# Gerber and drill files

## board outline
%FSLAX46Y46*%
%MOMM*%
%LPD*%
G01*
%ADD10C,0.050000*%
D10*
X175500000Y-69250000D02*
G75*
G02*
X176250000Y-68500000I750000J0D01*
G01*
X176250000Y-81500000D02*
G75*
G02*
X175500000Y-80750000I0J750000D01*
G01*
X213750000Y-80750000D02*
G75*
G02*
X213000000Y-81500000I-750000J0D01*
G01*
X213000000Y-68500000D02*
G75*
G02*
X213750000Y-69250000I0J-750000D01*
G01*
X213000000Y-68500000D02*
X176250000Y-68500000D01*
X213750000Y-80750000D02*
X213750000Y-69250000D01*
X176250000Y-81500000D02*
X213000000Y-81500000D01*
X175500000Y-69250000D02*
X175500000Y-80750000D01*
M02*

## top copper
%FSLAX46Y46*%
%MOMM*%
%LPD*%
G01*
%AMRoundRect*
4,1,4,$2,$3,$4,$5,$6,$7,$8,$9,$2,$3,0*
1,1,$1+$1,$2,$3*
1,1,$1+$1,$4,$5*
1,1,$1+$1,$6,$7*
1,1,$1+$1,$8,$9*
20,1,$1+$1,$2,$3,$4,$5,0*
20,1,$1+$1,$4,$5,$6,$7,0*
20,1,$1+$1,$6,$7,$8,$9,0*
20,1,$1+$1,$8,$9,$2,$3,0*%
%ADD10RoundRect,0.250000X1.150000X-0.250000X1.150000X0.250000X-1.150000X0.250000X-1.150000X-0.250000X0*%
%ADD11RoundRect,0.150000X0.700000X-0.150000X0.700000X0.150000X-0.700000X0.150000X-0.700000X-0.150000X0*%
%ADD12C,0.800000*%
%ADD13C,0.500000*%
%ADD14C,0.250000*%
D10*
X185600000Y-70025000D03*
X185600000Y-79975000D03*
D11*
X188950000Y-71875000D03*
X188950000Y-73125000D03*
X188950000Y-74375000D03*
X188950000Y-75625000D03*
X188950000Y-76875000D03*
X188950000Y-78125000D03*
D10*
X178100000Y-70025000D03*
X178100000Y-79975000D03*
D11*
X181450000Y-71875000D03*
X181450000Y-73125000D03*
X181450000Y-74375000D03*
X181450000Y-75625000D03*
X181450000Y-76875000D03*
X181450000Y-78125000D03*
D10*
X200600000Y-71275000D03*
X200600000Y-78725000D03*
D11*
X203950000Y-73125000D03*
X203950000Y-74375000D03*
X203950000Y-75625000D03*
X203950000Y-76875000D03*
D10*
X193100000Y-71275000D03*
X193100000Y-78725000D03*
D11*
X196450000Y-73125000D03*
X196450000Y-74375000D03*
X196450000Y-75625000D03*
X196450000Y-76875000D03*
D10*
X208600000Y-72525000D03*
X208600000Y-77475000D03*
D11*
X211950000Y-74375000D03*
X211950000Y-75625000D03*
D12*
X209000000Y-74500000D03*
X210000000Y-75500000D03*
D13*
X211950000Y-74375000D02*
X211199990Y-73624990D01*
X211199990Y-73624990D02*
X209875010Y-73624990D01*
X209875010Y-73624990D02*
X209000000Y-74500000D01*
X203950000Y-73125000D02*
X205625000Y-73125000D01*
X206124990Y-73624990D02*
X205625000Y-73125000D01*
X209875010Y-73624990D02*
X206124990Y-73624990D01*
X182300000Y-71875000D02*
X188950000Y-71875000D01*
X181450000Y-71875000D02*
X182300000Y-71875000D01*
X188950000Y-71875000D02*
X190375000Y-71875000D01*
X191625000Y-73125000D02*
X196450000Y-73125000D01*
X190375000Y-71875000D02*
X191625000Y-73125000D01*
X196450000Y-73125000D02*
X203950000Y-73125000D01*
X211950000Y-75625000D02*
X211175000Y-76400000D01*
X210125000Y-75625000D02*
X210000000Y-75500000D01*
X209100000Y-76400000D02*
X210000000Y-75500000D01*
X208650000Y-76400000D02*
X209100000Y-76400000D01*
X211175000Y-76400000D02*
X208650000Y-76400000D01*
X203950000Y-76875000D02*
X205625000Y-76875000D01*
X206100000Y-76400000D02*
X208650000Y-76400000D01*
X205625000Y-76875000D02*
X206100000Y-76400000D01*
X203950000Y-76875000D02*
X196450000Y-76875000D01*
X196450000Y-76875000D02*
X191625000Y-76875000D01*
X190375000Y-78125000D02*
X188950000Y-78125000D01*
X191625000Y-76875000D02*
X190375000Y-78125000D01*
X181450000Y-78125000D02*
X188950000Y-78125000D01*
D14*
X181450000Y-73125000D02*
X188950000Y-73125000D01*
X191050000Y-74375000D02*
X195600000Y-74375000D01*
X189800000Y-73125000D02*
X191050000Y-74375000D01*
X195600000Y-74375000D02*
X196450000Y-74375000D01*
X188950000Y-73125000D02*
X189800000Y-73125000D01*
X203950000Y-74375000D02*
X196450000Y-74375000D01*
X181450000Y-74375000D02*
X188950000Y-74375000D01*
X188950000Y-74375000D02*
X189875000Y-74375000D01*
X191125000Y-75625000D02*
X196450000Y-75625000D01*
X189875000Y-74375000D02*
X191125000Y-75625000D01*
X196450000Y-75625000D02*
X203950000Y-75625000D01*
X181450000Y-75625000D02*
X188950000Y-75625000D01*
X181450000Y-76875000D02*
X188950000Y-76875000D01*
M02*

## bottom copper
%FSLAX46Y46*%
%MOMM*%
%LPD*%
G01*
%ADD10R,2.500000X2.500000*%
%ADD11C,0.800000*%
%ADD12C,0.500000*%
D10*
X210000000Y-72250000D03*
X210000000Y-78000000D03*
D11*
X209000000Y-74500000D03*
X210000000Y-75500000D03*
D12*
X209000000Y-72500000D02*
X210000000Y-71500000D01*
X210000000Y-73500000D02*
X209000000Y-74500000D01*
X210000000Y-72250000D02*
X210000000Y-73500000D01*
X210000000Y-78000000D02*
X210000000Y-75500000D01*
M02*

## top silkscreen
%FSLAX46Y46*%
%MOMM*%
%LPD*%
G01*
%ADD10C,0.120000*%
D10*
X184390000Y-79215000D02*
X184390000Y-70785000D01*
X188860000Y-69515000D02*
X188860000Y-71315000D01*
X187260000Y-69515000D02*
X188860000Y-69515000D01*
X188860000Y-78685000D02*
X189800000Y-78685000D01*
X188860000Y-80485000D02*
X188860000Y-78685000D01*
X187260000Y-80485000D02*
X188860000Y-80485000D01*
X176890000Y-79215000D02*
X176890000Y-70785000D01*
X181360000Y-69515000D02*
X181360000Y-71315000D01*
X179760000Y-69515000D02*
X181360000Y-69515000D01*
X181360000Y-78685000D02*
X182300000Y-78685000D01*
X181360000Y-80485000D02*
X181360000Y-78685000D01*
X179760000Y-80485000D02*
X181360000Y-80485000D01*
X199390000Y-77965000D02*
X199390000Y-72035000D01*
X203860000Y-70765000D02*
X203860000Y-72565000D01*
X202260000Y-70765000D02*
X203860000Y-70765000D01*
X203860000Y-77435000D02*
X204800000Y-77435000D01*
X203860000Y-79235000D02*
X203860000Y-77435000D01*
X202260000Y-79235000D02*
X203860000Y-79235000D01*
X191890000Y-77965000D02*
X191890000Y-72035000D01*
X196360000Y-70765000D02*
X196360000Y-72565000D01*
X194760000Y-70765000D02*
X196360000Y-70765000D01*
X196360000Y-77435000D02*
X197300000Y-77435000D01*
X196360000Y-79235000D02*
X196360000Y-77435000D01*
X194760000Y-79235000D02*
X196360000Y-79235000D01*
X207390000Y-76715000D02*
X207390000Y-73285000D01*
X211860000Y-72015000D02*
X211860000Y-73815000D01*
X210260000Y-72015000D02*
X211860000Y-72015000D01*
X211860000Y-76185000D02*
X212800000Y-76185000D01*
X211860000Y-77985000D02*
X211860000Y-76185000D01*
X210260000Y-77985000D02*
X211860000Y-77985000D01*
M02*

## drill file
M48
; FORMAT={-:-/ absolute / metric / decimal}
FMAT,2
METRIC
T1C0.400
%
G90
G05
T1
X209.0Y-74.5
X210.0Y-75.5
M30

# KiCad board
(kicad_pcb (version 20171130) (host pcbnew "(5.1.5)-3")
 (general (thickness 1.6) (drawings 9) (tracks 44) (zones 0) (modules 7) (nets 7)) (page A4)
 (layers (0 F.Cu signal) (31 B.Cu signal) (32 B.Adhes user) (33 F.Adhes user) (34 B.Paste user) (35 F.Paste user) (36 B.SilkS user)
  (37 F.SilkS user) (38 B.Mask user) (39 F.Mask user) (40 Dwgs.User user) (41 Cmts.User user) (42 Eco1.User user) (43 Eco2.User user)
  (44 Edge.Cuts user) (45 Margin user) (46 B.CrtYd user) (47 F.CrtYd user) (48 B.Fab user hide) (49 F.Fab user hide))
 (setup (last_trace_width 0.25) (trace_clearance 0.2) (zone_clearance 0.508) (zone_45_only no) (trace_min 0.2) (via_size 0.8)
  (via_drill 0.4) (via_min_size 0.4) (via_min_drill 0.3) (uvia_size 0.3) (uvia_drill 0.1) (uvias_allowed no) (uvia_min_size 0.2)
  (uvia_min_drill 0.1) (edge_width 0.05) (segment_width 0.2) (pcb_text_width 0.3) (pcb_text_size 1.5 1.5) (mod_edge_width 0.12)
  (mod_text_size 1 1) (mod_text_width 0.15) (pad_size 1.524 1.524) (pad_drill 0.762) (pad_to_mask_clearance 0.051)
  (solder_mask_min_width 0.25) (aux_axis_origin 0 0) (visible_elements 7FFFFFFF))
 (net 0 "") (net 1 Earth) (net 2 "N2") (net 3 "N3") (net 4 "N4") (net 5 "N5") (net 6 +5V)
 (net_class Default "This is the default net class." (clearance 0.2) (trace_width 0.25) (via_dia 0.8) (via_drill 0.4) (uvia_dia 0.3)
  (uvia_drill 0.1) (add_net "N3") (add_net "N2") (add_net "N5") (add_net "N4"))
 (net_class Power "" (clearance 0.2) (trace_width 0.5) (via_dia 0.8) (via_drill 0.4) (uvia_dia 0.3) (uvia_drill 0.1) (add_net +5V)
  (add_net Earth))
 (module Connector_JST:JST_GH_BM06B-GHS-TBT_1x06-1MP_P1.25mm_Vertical (layer F.Cu) (at 187 75 90)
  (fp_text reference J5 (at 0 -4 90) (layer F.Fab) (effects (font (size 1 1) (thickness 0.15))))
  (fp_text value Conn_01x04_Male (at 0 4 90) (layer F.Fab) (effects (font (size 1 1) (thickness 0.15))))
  (fp_line (start -4.215 -2.61) (end 4.215 -2.61) (layer F.SilkS) (width 0.12))
  (fp_line (start 5.485 1.86) (end 3.685 1.86) (layer F.SilkS) (width 0.12))
  (fp_line (start 5.485 0.26) (end 5.485 1.86) (layer F.SilkS) (width 0.12))
  (fp_line (start -3.685 1.86) (end -3.685 2.8) (layer F.SilkS) (width 0.12))
  (fp_line (start -5.485 1.86) (end -3.685 1.86) (layer F.SilkS) (width 0.12))
  (fp_line (start -5.485 0.26) (end -5.485 1.86) (layer F.SilkS) (width 0.12))
  (pad MP smd roundrect (at 4.975 -1.4 90) (size 1 2.8) (layers F.Cu F.Paste F.Mask) (roundrect_rratio 0.25))
  (pad MP smd roundrect (at -4.975 -1.4 90) (size 1 2.8) (layers F.Cu F.Paste F.Mask) (roundrect_rratio 0.25))
  (pad 6 smd roundrect (at 3.125 1.95 90) (size 0.6 1.7) (layers F.Cu F.Paste F.Mask) (roundrect_rratio 0.25) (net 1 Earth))
  (pad 5 smd roundrect (at 1.875 1.95 90) (size 0.6 1.7) (layers F.Cu F.Paste F.Mask) (roundrect_rratio 0.25) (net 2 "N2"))
  (pad 4 smd roundrect (at 0.625 1.95 90) (size 0.6 1.7) (layers F.Cu F.Paste F.Mask) (roundrect_rratio 0.25) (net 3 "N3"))
  (pad 3 smd roundrect (at -0.625 1.95 90) (size 0.6 1.7) (layers F.Cu F.Paste F.Mask) (roundrect_rratio 0.25) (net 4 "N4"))
  (pad 2 smd roundrect (at -1.875 1.95 90) (size 0.6 1.7) (layers F.Cu F.Paste F.Mask) (roundrect_rratio 0.25) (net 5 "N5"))
  (pad 1 smd roundrect (at -3.125 1.95 90) (size 0.6 1.7) (layers F.Cu F.Paste F.Mask) (roundrect_rratio 0.25) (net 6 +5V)))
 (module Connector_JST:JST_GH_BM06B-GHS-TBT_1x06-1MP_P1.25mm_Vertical (layer F.Cu) (at 179.5 75 90)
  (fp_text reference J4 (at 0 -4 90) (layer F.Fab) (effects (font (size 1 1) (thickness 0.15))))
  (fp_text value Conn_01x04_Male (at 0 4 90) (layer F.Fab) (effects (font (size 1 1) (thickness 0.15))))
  (fp_line (start -4.215 -2.61) (end 4.215 -2.61) (layer F.SilkS) (width 0.12))
  (fp_line (start 5.485 1.86) (end 3.685 1.86) (layer F.SilkS) (width 0.12))
  (fp_line (start 5.485 0.26) (end 5.485 1.86) (layer F.SilkS) (width 0.12))
  (fp_line (start -3.685 1.86) (end -3.685 2.8) (layer F.SilkS) (width 0.12))
  (fp_line (start -5.485 1.86) (end -3.685 1.86) (layer F.SilkS) (width 0.12))
  (fp_line (start -5.485 0.26) (end -5.485 1.86) (layer F.SilkS) (width 0.12))
  (pad MP smd roundrect (at 4.975 -1.4 90) (size 1 2.8) (layers F.Cu F.Paste F.Mask) (roundrect_rratio 0.25))
  (pad MP smd roundrect (at -4.975 -1.4 90) (size 1 2.8) (layers F.Cu F.Paste F.Mask) (roundrect_rratio 0.25))
  (pad 6 smd roundrect (at 3.125 1.95 90) (size 0.6 1.7) (layers F.Cu F.Paste F.Mask) (roundrect_rratio 0.25) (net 1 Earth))
  (pad 5 smd roundrect (at 1.875 1.95 90) (size 0.6 1.7) (layers F.Cu F.Paste F.Mask) (roundrect_rratio 0.25) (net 2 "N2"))
  (pad 4 smd roundrect (at 0.625 1.95 90) (size 0.6 1.7) (layers F.Cu F.Paste F.Mask) (roundrect_rratio 0.25) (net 3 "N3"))
  (pad 3 smd roundrect (at -0.625 1.95 90) (size 0.6 1.7) (layers F.Cu F.Paste F.Mask) (roundrect_rratio 0.25) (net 4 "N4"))
  (pad 2 smd roundrect (at -1.875 1.95 90) (size 0.6 1.7) (layers F.Cu F.Paste F.Mask) (roundrect_rratio 0.25) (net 5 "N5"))
  (pad 1 smd roundrect (at -3.125 1.95 90) (size 0.6 1.7) (layers F.Cu F.Paste F.Mask) (roundrect_rratio 0.25) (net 6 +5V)))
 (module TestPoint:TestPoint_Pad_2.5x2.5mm (layer B.Cu) (at 210 72.25)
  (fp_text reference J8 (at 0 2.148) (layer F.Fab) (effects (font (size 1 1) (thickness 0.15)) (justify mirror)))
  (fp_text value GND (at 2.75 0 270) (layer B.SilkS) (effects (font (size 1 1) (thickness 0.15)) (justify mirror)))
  (pad 1 smd rect (at 0 0) (size 2.5 2.5) (layers B.Cu B.Mask) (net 1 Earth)))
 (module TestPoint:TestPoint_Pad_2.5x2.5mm (layer B.Cu) (at 210 78)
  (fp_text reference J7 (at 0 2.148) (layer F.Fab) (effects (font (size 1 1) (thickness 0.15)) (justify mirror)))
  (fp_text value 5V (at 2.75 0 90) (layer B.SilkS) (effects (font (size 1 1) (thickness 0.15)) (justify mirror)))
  (pad 1 smd rect (at 0 0) (size 2.5 2.5) (layers B.Cu B.Mask) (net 6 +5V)))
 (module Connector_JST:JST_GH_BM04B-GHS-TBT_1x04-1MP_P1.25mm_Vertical (layer F.Cu) (at 202 75 90)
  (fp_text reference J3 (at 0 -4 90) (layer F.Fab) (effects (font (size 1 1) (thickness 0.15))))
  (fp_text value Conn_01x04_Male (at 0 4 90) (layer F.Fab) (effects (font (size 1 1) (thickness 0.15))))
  (fp_line (start -2.965 -2.61) (end 2.965 -2.61) (layer F.SilkS) (width 0.12))
  (fp_line (start 4.235 1.86) (end 2.435 1.86) (layer F.SilkS) (width 0.12))
  (fp_line (start 4.235 0.26) (end 4.235 1.86) (layer F.SilkS) (width 0.12))
  (fp_line (start -2.435 1.86) (end -2.435 2.8) (layer F.SilkS) (width 0.12))
  (fp_line (start -4.235 1.86) (end -2.435 1.86) (layer F.SilkS) (width 0.12))
  (fp_line (start -4.235 0.26) (end -4.235 1.86) (layer F.SilkS) (width 0.12))
  (pad MP smd roundrect (at 3.725 -1.4 90) (size 1 2.8) (layers F.Cu F.Paste F.Mask) (roundrect_rratio 0.25))
  (pad MP smd roundrect (at -3.725 -1.4 90) (size 1 2.8) (layers F.Cu F.Paste F.Mask) (roundrect_rratio 0.25))
  (pad 4 smd roundrect (at 1.875 1.95 90) (size 0.6 1.7) (layers F.Cu F.Paste F.Mask) (roundrect_rratio 0.25) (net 1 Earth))
  (pad 3 smd roundrect (at 0.625 1.95 90) (size 0.6 1.7) (layers F.Cu F.Paste F.Mask) (roundrect_rratio 0.25) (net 2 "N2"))
  (pad 2 smd roundrect (at -0.625 1.95 90) (size 0.6 1.7) (layers F.Cu F.Paste F.Mask) (roundrect_rratio 0.25) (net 3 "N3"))
  (pad 1 smd roundrect (at -1.875 1.95 90) (size 0.6 1.7) (layers F.Cu F.Paste F.Mask) (roundrect_rratio 0.25) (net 6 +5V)))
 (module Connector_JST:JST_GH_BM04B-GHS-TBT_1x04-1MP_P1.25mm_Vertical (layer F.Cu) (at 194.5 75 90)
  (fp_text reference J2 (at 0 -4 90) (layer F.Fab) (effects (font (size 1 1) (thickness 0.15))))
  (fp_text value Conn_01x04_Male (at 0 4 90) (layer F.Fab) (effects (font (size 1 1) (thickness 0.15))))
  (fp_line (start -2.965 -2.61) (end 2.965 -2.61) (layer F.SilkS) (width 0.12))
  (fp_line (start 4.235 1.86) (end 2.435 1.86) (layer F.SilkS) (width 0.12))
  (fp_line (start 4.235 0.26) (end 4.235 1.86) (layer F.SilkS) (width 0.12))
  (fp_line (start -2.435 1.86) (end -2.435 2.8) (layer F.SilkS) (width 0.12))
  (fp_line (start -4.235 1.86) (end -2.435 1.86) (layer F.SilkS) (width 0.12))
  (fp_line (start -4.235 0.26) (end -4.235 1.86) (layer F.SilkS) (width 0.12))
  (pad MP smd roundrect (at 3.725 -1.4 90) (size 1 2.8) (layers F.Cu F.Paste F.Mask) (roundrect_rratio 0.25))
  (pad MP smd roundrect (at -3.725 -1.4 90) (size 1 2.8) (layers F.Cu F.Paste F.Mask) (roundrect_rratio 0.25))
  (pad 4 smd roundrect (at 1.875 1.95 90) (size 0.6 1.7) (layers F.Cu F.Paste F.Mask) (roundrect_rratio 0.25) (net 1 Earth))
  (pad 3 smd roundrect (at 0.625 1.95 90) (size 0.6 1.7) (layers F.Cu F.Paste F.Mask) (roundrect_rratio 0.25) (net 2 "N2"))
  (pad 2 smd roundrect (at -0.625 1.95 90) (size 0.6 1.7) (layers F.Cu F.Paste F.Mask) (roundrect_rratio 0.25) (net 3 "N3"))
  (pad 1 smd roundrect (at -1.875 1.95 90) (size 0.6 1.7) (layers F.Cu F.Paste F.Mask) (roundrect_rratio 0.25) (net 6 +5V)))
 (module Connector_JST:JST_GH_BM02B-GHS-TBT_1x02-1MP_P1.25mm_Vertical (layer F.Cu) (at 210 75 90)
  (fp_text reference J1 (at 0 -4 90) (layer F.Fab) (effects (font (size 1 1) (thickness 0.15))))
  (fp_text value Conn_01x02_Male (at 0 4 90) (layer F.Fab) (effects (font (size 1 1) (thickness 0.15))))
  (fp_line (start -1.715 -2.61) (end 1.715 -2.61) (layer F.SilkS) (width 0.12))
  (fp_line (start 2.985 1.86) (end 1.185 1.86) (layer F.SilkS) (width 0.12))
  (fp_line (start 2.985 0.26) (end 2.985 1.86) (layer F.SilkS) (width 0.12))
  (fp_line (start -1.185 1.86) (end -1.185 2.8) (layer F.SilkS) (width 0.12))
  (fp_line (start -2.985 1.86) (end -1.185 1.86) (layer F.SilkS) (width 0.12))
  (fp_line (start -2.985 0.26) (end -2.985 1.86) (layer F.SilkS) (width 0.12))
  (pad MP smd roundrect (at 2.475 -1.4 90) (size 1 2.8) (layers F.Cu F.Paste F.Mask) (roundrect_rratio 0.25))
  (pad MP smd roundrect (at -2.475 -1.4 90) (size 1 2.8) (layers F.Cu F.Paste F.Mask) (roundrect_rratio 0.25))
  (pad 2 smd roundrect (at 0.625 1.95 90) (size 0.6 1.7) (layers F.Cu F.Paste F.Mask) (roundrect_rratio 0.25) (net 1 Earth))
  (pad 1 smd roundrect (at -0.625 1.95 90) (size 0.6 1.7) (layers F.Cu F.Paste F.Mask) (roundrect_rratio 0.25) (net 6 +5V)))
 (gr_arc (start 176.25 69.25) (end 176.25 68.5) (angle -90) (layer Edge.Cuts) (width 0.05))
 (gr_arc (start 176.25 80.75) (end 175.5 80.75) (angle -90) (layer Edge.Cuts) (width 0.05))
 (gr_arc (start 213 80.75) (end 213 81.5) (angle -90) (layer Edge.Cuts) (width 0.05))
 (gr_arc (start 213 69.25) (end 213.75 69.25) (angle -90) (layer Edge.Cuts) (width 0.05))
 (gr_line (start 213 68.5) (end 176.25 68.5) (layer Edge.Cuts) (width 0.05))
 (gr_line (start 213.75 80.75) (end 213.75 69.25) (layer Edge.Cuts) (width 0.05))
 (gr_line (start 176.25 81.5) (end 213 81.5) (layer Edge.Cuts) (width 0.05))
 (gr_line (start 175.5 69.25) (end 175.5 80.75) (layer Edge.Cuts) (width 0.05))
 (segment (start 211.95 74.375) (end 211.19999 73.62499) (width 0.5) (layer F.Cu) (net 1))
 (segment (start 211.19999 73.62499) (end 209.87501 73.62499) (width 0.5) (layer F.Cu) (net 1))
 (via (at 209 74.5) (size 0.8) (drill 0.4) (layers F.Cu B.Cu) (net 1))
 (segment (start 209.87501 73.62499) (end 209 74.5) (width 0.5) (layer F.Cu) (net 1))
 (segment (start 209 72.5) (end 210 71.5) (width 0.5) (layer B.Cu) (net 1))
 (segment (start 210 73.5) (end 209 74.5) (width 0.5) (layer B.Cu) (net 1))
 (segment (start 210 72.25) (end 210 73.5) (width 0.5) (layer B.Cu) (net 1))
 (segment (start 203.95 73.125) (end 205.625 73.125) (width 0.5) (layer F.Cu) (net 1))
 (segment (start 206.12499 73.62499) (end 205.625 73.125) (width 0.5) (layer F.Cu) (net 1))
 (segment (start 209.87501 73.62499) (end 206.12499 73.62499) (width 0.5) (layer F.Cu) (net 1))
 (segment (start 182.3 71.875) (end 188.95 71.875) (width 0.5) (layer F.Cu) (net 1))
 (segment (start 181.45 71.875) (end 182.3 71.875) (width 0.5) (layer F.Cu) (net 1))
 (segment (start 188.95 71.875) (end 190.375 71.875) (width 0.5) (layer F.Cu) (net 1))
 (segment (start 191.625 73.125) (end 196.45 73.125) (width 0.5) (layer F.Cu) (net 1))
 (segment (start 190.375 71.875) (end 191.625 73.125) (width 0.5) (layer F.Cu) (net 1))
 (segment (start 196.45 73.125) (end 203.95 73.125) (width 0.5) (layer F.Cu) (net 1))
 (segment (start 211.95 75.625) (end 211.175 76.4) (width 0.5) (layer F.Cu) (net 6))
 (via (at 210 75.5) (size 0.8) (drill 0.4) (layers F.Cu B.Cu) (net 6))
 (segment (start 210.125 75.625) (end 210 75.5) (width 0.5) (layer F.Cu) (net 6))
 (segment (start 209.1 76.4) (end 210 75.5) (width 0.5) (layer F.Cu) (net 6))
 (segment (start 208.65 76.4) (end 209.1 76.4) (width 0.5) (layer F.Cu) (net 6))
 (segment (start 211.175 76.4) (end 208.65 76.4) (width 0.5) (layer F.Cu) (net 6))
 (segment (start 210 78) (end 210 75.5) (width 0.5) (layer B.Cu) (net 6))
 (segment (start 203.95 76.875) (end 205.625 76.875) (width 0.5) (layer F.Cu) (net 6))
 (segment (start 206.1 76.4) (end 208.65 76.4) (width 0.5) (layer F.Cu) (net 6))
 (segment (start 205.625 76.875) (end 206.1 76.4) (width 0.5) (layer F.Cu) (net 6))
 (segment (start 203.95 76.875) (end 196.45 76.875) (width 0.5) (layer F.Cu) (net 6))
 (segment (start 196.45 76.875) (end 191.625 76.875) (width 0.5) (layer F.Cu) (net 6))
 (segment (start 190.375 78.125) (end 188.95 78.125) (width 0.5) (layer F.Cu) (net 6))
 (segment (start 191.625 76.875) (end 190.375 78.125) (width 0.5) (layer F.Cu) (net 6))
 (segment (start 181.45 78.125) (end 188.95 78.125) (width 0.5) (layer F.Cu) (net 6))
 (segment (start 181.45 73.125) (end 188.95 73.125) (width 0.25) (layer F.Cu) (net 2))
 (segment (start 191.05 74.375) (end 195.6 74.375) (width 0.25) (layer F.Cu) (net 2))
 (segment (start 189.8 73.125) (end 191.05 74.375) (width 0.25) (layer F.Cu) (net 2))
 (segment (start 195.6 74.375) (end 196.45 74.375) (width 0.25) (layer F.Cu) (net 2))
 (segment (start 188.95 73.125) (end 189.8 73.125) (width 0.25) (layer F.Cu) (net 2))
 (segment (start 203.95 74.375) (end 196.45 74.375) (width 0.25) (layer F.Cu) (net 2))
 (segment (start 181.45 74.375) (end 188.95 74.375) (width 0.25) (layer F.Cu) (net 3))
 (segment (start 188.95 74.375) (end 189.875 74.375) (width 0.25) (layer F.Cu) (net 3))
 (segment (start 191.125 75.625) (end 196.45 75.625) (width 0.25) (layer F.Cu) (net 3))
 (segment (start 189.875 74.375) (end 191.125 75.625) (width 0.25) (layer F.Cu) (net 3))
 (segment (start 196.45 75.625) (end 203.95 75.625) (width 0.25) (layer F.Cu) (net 3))
 (segment (start 181.45 75.625) (end 188.95 75.625) (width 0.25) (layer F.Cu) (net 4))
 (segment (start 181.45 76.875) (end 188.95 76.875) (width 0.25) (layer F.Cu) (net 5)))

